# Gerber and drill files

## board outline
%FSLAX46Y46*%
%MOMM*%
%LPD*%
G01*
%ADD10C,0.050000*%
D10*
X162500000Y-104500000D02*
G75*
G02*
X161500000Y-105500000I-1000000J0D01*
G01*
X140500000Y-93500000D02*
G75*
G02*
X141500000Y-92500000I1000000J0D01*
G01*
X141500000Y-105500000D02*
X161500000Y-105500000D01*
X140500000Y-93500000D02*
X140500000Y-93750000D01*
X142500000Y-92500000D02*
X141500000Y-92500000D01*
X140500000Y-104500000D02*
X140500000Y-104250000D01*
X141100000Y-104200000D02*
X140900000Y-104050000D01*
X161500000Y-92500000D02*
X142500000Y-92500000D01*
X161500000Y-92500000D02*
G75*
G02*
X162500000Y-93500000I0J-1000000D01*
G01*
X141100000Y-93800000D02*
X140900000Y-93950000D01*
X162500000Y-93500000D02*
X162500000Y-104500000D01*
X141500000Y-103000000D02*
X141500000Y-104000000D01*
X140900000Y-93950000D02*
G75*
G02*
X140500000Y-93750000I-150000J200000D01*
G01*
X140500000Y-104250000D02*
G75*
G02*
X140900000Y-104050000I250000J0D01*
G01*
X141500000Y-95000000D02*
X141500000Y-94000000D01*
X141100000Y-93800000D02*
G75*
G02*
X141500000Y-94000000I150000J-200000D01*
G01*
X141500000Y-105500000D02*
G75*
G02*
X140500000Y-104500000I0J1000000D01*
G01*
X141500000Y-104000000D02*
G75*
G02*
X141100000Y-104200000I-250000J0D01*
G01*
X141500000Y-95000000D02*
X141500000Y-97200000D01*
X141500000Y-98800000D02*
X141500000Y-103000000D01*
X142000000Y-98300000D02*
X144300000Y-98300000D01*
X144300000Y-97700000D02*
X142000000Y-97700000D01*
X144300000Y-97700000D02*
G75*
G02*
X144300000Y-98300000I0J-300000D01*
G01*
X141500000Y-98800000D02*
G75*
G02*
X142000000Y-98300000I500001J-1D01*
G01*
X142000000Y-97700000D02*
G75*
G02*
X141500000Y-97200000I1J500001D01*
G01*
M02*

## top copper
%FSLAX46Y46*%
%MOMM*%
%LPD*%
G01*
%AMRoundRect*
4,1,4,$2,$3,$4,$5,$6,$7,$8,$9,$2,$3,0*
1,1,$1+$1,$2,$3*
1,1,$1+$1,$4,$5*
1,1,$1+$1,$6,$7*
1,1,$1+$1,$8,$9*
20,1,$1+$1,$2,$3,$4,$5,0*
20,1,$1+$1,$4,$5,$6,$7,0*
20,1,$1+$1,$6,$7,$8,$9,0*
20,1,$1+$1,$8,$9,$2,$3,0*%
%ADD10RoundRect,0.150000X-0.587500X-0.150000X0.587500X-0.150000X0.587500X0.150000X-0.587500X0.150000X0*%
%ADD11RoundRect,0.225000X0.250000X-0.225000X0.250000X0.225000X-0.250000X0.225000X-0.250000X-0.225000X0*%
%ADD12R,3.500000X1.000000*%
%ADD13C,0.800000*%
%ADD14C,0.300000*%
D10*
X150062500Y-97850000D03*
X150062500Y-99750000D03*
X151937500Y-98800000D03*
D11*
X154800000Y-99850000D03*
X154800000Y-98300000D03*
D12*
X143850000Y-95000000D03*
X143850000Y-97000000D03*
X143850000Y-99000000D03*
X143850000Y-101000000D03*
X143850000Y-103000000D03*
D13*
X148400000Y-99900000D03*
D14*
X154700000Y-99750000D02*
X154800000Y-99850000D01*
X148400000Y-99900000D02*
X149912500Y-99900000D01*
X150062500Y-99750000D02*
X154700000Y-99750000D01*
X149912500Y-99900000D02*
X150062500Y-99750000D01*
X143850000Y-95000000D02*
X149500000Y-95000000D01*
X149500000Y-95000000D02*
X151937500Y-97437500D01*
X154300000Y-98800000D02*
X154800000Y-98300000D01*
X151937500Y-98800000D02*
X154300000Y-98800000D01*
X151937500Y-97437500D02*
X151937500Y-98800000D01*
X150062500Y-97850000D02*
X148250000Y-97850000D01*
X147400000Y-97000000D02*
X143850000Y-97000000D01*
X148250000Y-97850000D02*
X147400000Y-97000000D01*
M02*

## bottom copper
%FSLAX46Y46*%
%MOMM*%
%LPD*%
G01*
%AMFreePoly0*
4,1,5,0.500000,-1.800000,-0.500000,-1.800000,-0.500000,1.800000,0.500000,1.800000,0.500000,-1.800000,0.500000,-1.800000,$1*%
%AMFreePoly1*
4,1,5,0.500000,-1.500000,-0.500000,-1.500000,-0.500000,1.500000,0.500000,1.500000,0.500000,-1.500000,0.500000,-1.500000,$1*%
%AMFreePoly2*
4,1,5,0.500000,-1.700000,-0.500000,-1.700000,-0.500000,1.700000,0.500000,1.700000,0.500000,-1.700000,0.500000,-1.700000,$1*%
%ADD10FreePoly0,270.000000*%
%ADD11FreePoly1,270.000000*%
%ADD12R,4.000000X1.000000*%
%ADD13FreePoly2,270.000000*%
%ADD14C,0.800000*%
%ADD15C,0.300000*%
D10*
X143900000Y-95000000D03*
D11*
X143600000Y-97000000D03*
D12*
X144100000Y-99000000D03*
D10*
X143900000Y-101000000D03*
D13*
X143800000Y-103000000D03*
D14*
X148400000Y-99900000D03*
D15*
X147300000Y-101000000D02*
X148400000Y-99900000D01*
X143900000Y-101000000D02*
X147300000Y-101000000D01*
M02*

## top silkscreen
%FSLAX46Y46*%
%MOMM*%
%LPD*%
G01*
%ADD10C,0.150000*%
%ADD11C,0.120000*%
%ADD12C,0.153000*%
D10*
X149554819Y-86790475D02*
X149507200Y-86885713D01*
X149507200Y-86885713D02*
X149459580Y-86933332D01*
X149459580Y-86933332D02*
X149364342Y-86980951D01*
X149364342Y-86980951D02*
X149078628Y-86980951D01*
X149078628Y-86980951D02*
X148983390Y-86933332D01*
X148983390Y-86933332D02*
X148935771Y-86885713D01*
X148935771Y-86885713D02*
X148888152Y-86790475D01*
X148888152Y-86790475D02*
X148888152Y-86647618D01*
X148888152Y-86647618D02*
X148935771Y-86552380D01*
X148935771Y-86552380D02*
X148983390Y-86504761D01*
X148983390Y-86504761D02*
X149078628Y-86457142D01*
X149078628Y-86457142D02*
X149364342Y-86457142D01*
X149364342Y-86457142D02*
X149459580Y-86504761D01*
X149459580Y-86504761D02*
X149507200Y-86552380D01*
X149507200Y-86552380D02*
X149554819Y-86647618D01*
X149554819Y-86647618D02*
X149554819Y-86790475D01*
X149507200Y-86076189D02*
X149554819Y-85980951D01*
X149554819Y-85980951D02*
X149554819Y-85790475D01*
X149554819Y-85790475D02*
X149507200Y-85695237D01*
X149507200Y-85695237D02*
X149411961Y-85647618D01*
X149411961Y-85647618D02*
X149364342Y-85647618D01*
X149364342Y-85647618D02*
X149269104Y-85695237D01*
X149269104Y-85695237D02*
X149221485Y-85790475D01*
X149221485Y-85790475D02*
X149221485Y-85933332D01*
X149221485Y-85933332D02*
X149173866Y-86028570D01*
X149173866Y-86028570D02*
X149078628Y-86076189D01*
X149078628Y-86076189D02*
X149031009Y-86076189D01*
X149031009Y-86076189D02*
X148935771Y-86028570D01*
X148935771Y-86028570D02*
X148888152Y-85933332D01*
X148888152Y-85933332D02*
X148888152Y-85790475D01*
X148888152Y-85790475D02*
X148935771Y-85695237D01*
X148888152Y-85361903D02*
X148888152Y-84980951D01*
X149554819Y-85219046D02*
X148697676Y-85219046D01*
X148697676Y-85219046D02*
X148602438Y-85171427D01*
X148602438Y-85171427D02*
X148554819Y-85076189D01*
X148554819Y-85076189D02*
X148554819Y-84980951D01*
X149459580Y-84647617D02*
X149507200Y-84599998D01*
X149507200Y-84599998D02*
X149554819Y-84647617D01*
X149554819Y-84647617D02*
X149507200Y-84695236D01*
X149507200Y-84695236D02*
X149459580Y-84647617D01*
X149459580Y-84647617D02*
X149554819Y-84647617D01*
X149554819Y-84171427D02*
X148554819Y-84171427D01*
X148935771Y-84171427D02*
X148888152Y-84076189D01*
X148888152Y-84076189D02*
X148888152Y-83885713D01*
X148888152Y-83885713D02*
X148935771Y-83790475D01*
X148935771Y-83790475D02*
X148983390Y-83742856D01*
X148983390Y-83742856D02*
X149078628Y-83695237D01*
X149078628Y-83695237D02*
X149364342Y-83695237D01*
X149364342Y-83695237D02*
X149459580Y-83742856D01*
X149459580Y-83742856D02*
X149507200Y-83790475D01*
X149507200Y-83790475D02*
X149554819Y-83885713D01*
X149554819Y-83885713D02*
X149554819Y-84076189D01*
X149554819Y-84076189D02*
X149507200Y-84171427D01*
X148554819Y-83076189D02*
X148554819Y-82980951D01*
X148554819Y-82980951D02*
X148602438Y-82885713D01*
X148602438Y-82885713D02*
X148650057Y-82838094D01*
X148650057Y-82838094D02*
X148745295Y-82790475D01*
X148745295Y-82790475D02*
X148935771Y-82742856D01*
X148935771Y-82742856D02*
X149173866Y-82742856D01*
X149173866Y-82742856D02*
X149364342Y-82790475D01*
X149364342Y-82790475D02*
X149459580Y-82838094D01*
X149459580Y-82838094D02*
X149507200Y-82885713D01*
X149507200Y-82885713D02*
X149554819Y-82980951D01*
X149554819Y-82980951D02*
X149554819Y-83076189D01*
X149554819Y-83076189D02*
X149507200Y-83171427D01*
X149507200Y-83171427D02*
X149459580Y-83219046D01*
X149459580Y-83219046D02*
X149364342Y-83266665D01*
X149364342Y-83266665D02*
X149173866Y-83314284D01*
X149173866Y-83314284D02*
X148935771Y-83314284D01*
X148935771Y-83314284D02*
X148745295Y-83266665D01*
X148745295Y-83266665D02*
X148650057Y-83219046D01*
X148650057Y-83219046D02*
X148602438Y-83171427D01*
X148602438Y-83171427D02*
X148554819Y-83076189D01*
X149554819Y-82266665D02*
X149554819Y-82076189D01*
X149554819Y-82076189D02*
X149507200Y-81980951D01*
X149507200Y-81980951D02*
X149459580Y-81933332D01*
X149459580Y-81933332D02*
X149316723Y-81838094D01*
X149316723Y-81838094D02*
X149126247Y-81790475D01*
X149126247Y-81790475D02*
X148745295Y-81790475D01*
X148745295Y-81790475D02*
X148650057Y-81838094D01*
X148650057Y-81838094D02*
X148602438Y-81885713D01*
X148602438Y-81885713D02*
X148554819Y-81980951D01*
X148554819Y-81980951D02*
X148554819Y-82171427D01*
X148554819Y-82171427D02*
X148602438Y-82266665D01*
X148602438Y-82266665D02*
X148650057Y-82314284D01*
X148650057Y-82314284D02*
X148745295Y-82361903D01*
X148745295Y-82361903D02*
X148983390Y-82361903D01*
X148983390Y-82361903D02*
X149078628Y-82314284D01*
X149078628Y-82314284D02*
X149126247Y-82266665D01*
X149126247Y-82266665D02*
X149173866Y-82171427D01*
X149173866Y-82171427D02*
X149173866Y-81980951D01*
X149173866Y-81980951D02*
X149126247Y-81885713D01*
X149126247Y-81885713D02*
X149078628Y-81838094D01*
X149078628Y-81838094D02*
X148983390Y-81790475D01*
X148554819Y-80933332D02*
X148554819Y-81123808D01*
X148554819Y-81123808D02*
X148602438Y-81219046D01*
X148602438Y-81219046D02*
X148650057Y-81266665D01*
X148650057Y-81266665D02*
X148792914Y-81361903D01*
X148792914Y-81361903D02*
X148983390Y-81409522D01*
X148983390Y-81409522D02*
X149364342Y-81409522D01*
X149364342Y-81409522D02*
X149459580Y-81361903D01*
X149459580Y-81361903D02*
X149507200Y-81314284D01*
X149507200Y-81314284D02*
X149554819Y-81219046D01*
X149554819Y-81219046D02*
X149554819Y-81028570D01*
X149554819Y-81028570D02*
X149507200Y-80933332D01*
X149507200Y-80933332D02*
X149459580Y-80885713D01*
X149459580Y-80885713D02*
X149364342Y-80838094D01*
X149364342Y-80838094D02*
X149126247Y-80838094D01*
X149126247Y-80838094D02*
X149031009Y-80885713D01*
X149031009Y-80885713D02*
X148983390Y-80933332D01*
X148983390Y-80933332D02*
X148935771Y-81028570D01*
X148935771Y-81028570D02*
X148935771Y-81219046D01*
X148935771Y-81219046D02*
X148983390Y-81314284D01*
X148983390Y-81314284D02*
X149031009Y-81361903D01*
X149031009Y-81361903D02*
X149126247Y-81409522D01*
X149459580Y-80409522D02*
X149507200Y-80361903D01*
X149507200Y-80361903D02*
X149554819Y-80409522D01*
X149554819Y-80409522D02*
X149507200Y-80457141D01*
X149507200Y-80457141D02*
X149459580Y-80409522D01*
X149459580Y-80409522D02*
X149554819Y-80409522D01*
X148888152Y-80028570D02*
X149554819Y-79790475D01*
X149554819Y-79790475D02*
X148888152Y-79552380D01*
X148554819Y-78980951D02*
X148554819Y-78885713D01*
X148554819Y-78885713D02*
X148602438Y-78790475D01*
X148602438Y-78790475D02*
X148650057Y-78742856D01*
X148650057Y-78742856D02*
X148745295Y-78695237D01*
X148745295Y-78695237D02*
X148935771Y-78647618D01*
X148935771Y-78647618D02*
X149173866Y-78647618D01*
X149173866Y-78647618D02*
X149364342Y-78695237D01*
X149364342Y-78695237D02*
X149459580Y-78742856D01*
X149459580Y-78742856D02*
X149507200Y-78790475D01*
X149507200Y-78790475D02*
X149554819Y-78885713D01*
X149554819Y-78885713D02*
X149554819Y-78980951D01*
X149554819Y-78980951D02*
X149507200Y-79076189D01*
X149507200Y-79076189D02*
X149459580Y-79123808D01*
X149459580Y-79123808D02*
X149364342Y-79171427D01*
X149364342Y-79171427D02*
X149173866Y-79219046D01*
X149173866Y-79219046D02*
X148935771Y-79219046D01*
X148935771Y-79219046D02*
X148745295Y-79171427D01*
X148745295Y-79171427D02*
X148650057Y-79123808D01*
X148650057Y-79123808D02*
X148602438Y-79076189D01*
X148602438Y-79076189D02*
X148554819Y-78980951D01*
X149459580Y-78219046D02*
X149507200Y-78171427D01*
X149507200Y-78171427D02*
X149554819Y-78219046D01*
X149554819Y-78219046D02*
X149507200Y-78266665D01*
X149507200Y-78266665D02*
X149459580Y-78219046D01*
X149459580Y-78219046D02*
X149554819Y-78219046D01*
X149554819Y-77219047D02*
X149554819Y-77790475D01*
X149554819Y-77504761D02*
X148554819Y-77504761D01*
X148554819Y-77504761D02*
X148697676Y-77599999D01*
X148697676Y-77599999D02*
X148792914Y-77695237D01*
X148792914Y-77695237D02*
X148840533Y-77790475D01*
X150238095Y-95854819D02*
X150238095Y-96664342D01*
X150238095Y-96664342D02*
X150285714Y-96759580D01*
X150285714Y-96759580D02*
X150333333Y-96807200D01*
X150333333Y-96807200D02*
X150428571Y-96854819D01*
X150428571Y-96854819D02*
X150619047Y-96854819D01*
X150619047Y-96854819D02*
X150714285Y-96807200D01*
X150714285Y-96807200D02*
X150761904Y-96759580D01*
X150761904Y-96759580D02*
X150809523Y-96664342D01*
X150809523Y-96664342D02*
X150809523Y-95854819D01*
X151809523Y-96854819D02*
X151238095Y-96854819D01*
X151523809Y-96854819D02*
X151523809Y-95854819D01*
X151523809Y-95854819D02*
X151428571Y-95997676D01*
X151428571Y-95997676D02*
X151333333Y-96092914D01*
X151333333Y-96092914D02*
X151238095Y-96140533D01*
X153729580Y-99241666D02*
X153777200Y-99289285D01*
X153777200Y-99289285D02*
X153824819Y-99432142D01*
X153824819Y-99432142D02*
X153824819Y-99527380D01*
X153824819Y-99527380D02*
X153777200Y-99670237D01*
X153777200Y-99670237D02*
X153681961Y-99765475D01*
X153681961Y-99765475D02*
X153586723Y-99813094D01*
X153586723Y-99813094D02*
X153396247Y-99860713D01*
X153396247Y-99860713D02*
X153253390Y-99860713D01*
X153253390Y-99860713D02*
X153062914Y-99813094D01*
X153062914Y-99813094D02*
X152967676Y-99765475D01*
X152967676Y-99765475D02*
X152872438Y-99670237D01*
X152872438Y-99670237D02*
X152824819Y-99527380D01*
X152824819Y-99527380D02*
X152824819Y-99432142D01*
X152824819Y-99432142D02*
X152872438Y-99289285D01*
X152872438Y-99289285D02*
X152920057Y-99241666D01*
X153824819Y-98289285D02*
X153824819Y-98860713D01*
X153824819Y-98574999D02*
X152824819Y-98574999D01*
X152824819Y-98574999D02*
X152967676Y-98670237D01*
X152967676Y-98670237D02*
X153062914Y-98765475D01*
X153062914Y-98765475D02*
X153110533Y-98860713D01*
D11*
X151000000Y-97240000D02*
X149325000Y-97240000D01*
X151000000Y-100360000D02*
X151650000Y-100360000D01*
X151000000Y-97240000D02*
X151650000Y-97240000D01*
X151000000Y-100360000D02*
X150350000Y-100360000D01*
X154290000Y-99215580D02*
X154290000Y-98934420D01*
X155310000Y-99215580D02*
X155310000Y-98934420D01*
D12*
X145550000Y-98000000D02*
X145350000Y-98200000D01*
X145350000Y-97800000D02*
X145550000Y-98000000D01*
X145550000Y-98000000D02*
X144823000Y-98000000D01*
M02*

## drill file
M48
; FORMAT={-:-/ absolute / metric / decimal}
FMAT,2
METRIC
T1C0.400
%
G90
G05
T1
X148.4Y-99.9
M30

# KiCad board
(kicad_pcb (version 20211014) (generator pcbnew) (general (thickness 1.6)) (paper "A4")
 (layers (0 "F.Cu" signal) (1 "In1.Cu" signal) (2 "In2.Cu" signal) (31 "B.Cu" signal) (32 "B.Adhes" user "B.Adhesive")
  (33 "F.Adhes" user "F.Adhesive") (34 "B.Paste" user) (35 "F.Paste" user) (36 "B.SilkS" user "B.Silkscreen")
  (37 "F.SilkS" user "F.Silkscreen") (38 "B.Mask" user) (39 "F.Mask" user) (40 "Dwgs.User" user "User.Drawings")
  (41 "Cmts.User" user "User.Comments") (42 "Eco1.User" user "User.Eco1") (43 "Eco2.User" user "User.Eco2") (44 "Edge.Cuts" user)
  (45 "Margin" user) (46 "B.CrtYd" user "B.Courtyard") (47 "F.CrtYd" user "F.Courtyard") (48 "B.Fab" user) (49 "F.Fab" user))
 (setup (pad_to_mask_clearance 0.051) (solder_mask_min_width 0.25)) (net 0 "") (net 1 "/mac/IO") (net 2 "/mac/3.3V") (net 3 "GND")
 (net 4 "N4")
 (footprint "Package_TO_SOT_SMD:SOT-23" (layer "F.Cu") (at 151 98.8)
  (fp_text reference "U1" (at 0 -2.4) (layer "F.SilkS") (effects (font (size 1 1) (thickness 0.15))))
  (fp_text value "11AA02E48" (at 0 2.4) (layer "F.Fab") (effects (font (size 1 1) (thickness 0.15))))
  (fp_line (start 0 -1.56) (end -1.675 -1.56) (layer "F.SilkS") (width 0.12))
  (fp_line (start 0 1.56) (end 0.65 1.56) (layer "F.SilkS") (width 0.12))
  (fp_line (start 0 -1.56) (end 0.65 -1.56) (layer "F.SilkS") (width 0.12))
  (fp_line (start 0 1.56) (end -0.65 1.56) (layer "F.SilkS") (width 0.12))
  (pad "1" smd roundrect (at -0.9375 -0.95) (size 1.475 0.6) (layers "F.Cu" "F.Paste" "F.Mask") (roundrect_rratio 0.25) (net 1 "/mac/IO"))
  (pad "2" smd roundrect (at -0.9375 0.95) (size 1.475 0.6) (layers "F.Cu" "F.Paste" "F.Mask") (roundrect_rratio 0.25) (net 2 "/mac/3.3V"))
  (pad "3" smd roundrect (at 0.9375 0) (size 1.475 0.6) (layers "F.Cu" "F.Paste" "F.Mask") (roundrect_rratio 0.25) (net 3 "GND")))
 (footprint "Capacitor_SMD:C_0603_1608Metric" (layer "F.Cu") (at 154.8 99.075 90)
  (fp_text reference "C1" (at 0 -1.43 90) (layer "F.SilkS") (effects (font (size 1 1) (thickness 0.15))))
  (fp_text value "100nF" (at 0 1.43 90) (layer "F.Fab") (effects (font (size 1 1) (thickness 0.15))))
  (fp_line (start -0.14058 -0.51) (end 0.14058 -0.51) (layer "F.SilkS") (width 0.12))
  (fp_line (start -0.14058 0.51) (end 0.14058 0.51) (layer "F.SilkS") (width 0.12))
  (pad "1" smd roundrect (at -0.775 0 90) (size 0.9 0.95) (layers "F.Cu" "F.Paste" "F.Mask") (roundrect_rratio 0.25) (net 2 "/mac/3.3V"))
  (pad "2" smd roundrect (at 0.775 0 90) (size 0.9 0.95) (layers "F.Cu" "F.Paste" "F.Mask") (roundrect_rratio 0.25) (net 3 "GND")))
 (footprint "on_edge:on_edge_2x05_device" (layer "F.Cu") (at 141.5 99 -90)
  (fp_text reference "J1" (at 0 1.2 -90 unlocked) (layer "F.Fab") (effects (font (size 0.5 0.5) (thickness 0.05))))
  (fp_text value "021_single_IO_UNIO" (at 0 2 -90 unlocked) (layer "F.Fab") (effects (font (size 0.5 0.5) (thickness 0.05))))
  (fp_line (start -1 -4.05) (end -0.8 -3.85) (layer "F.SilkS") (width 0.153))
  (fp_line (start -1.2 -3.85) (end -1 -4.05) (layer "F.SilkS") (width 0.153))
  (fp_line (start -1 -4.05) (end -1 -3.323) (layer "F.SilkS") (width 0.153))
  (fp_line (start -4 0) (end -1.8 0) (layer "Edge.Cuts") (width 0.05))
  (fp_line (start -0.2 0) (end 4 0) (layer "Edge.Cuts") (width 0.05))
  (fp_line (start -0.7 -0.5) (end -0.7 -2.8) (layer "Edge.Cuts") (width 0.05))
  (fp_line (start -1.3 -2.8) (end -1.3 -0.5) (layer "Edge.Cuts") (width 0.05))
  (fp_arc (start -1.3 -2.8) (mid -1 -3.1) (end -0.7 -2.8) (layer "Edge.Cuts") (width 0.05))
  (fp_arc (start -0.2 0) (mid -0.553553 -0.146447) (end -0.7 -0.5) (layer "Edge.Cuts") (width 0.05))
  (fp_arc (start -1.3 -0.5) (mid -1.446447 -0.146447) (end -1.8 0) (layer "Edge.Cuts") (width 0.05))
  (pad "1" smd rect (at -4 -2.35 90) (size 1 3.5) (layers "F.Cu" "F.Mask") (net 3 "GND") (zone_connect 0))
  (pad "2" smd rect (at -2 -2.35 270) (size 1 3.5) (layers "F.Cu" "F.Mask") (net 1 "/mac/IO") (zone_connect 0))
  (pad "3" smd rect (at 0 -2.35 270) (size 1 3.5) (layers "F.Cu" "F.Mask") (zone_connect 0))
  (pad "4" smd rect (at 2 -2.35 90) (size 1 3.5) (layers "F.Cu" "F.Mask") (zone_connect 0))
  (pad "5" smd rect (at 4 -2.35 90) (size 1 3.5) (layers "F.Cu" "F.Mask") (zone_connect 0))
  (pad "6" smd custom (at -4 -2.4 270) (size 1 3.6) (layers "B.Cu" "B.Mask") (zone_connect 0) (options (clearance outline) (anchor rect))
   (primitives))
  (pad "7" smd custom (at -2 -2.1 270) (size 1 3) (layers "B.Cu" "B.Mask") (zone_connect 0) (options (clearance outline) (anchor rect))
   (primitives))
  (pad "8" smd rect (at 0 -2.6 270) (size 1 4) (layers "B.Cu" "B.Mask") (zone_connect 0))
  (pad "9" smd custom (at 2 -2.4 270) (size 1 3.6) (layers "B.Cu" "B.Mask") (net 2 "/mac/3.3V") (zone_connect 0)
   (options (clearance outline) (anchor rect)) (primitives))
  (pad "10" smd custom (at 4 -2.3 270) (size 1 3.4) (layers "B.Cu" "B.Mask") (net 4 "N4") (zone_connect 0)
   (options (clearance outline) (anchor rect)) (primitives)))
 (gr_arc (start 162.5 104.5) (mid 162.207107 105.207107) (end 161.5 105.5) (layer "Edge.Cuts") (width 0.05))
 (gr_arc (start 140.5 93.5) (mid 140.792893 92.792893) (end 141.5 92.5) (layer "Edge.Cuts") (width 0.05))
 (gr_line (start 141.5 105.5) (end 161.5 105.5) (layer "Edge.Cuts") (width 0.05))
 (gr_line (start 140.5 93.5) (end 140.5 93.75) (layer "Edge.Cuts") (width 0.05))
 (gr_line (start 142.5 92.5) (end 141.5 92.5) (layer "Edge.Cuts") (width 0.05))
 (gr_line (start 140.5 104.5) (end 140.5 104.25) (layer "Edge.Cuts") (width 0.05))
 (gr_line (start 141.1 104.2) (end 140.9 104.05) (layer "Edge.Cuts") (width 0.05))
 (gr_line (start 161.5 92.5) (end 142.5 92.5) (layer "Edge.Cuts") (width 0.05))
 (gr_arc (start 161.5 92.5) (mid 162.207107 92.792893) (end 162.5 93.5) (layer "Edge.Cuts") (width 0.05))
 (gr_line (start 141.1 93.8) (end 140.9 93.95) (layer "Edge.Cuts") (width 0.05))
 (gr_line (start 162.5 93.5) (end 162.5 104.5) (layer "Edge.Cuts") (width 0.05))
 (gr_line (start 141.5 103) (end 141.5 104) (layer "Edge.Cuts") (width 0.05))
 (gr_arc (start 140.9 93.95) (mid 140.638197 93.973607) (end 140.5 93.75) (layer "Edge.Cuts") (width 0.05))
 (gr_arc (start 140.5 104.25) (mid 140.638197 104.026393) (end 140.9 104.05) (layer "Edge.Cuts") (width 0.05))
 (gr_line (start 141.5 95) (end 141.5 94) (layer "Edge.Cuts") (width 0.05))
 (gr_arc (start 141.1 93.8) (mid 141.361803 93.776393) (end 141.5 94) (layer "Edge.Cuts") (width 0.05))
 (gr_arc (start 141.5 105.5) (mid 140.792893 105.207107) (end 140.5 104.5) (layer "Edge.Cuts") (width 0.05))
 (gr_arc (start 141.5 104) (mid 141.361803 104.223607) (end 141.1 104.2) (layer "Edge.Cuts") (width 0.05))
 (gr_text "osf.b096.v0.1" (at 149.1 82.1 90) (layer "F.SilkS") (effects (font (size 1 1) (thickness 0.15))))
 (segment (start 154.7 99.75) (end 154.8 99.85) (width 0.3) (layer "F.Cu") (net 2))
 (segment (start 148.4 99.9) (end 149.9125 99.9) (width 0.3) (layer "F.Cu") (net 2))
 (segment (start 150.0625 99.75) (end 154.7 99.75) (width 0.3) (layer "F.Cu") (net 2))
 (segment (start 149.9125 99.9) (end 150.0625 99.75) (width 0.3) (layer "F.Cu") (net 2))
 (via (at 148.4 99.9) (size 0.8) (drill 0.4) (layers "F.Cu" "B.Cu") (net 2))
 (segment (start 147.3 101) (end 148.4 99.9) (width 0.3) (layer "B.Cu") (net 2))
 (segment (start 143.9 101) (end 147.3 101) (width 0.3) (layer "B.Cu") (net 2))
 (segment (start 143.85 95) (end 149.5 95) (width 0.3) (layer "F.Cu") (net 3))
 (segment (start 149.5 95) (end 151.9375 97.4375) (width 0.3) (layer "F.Cu") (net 3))
 (segment (start 154.3 98.8) (end 154.8 98.3) (width 0.3) (layer "F.Cu") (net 3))
 (segment (start 151.9375 98.8) (end 154.3 98.8) (width 0.3) (layer "F.Cu") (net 3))
 (segment (start 151.9375 97.4375) (end 151.9375 98.8) (width 0.3) (layer "F.Cu") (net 3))
 (segment (start 150.0625 97.85) (end 148.25 97.85) (width 0.3) (layer "F.Cu") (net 1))
 (segment (start 147.4 97) (end 143.85 97) (width 0.3) (layer "F.Cu") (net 1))
 (segment (start 148.25 97.85) (end 147.4 97) (width 0.3) (layer "F.Cu") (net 1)))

